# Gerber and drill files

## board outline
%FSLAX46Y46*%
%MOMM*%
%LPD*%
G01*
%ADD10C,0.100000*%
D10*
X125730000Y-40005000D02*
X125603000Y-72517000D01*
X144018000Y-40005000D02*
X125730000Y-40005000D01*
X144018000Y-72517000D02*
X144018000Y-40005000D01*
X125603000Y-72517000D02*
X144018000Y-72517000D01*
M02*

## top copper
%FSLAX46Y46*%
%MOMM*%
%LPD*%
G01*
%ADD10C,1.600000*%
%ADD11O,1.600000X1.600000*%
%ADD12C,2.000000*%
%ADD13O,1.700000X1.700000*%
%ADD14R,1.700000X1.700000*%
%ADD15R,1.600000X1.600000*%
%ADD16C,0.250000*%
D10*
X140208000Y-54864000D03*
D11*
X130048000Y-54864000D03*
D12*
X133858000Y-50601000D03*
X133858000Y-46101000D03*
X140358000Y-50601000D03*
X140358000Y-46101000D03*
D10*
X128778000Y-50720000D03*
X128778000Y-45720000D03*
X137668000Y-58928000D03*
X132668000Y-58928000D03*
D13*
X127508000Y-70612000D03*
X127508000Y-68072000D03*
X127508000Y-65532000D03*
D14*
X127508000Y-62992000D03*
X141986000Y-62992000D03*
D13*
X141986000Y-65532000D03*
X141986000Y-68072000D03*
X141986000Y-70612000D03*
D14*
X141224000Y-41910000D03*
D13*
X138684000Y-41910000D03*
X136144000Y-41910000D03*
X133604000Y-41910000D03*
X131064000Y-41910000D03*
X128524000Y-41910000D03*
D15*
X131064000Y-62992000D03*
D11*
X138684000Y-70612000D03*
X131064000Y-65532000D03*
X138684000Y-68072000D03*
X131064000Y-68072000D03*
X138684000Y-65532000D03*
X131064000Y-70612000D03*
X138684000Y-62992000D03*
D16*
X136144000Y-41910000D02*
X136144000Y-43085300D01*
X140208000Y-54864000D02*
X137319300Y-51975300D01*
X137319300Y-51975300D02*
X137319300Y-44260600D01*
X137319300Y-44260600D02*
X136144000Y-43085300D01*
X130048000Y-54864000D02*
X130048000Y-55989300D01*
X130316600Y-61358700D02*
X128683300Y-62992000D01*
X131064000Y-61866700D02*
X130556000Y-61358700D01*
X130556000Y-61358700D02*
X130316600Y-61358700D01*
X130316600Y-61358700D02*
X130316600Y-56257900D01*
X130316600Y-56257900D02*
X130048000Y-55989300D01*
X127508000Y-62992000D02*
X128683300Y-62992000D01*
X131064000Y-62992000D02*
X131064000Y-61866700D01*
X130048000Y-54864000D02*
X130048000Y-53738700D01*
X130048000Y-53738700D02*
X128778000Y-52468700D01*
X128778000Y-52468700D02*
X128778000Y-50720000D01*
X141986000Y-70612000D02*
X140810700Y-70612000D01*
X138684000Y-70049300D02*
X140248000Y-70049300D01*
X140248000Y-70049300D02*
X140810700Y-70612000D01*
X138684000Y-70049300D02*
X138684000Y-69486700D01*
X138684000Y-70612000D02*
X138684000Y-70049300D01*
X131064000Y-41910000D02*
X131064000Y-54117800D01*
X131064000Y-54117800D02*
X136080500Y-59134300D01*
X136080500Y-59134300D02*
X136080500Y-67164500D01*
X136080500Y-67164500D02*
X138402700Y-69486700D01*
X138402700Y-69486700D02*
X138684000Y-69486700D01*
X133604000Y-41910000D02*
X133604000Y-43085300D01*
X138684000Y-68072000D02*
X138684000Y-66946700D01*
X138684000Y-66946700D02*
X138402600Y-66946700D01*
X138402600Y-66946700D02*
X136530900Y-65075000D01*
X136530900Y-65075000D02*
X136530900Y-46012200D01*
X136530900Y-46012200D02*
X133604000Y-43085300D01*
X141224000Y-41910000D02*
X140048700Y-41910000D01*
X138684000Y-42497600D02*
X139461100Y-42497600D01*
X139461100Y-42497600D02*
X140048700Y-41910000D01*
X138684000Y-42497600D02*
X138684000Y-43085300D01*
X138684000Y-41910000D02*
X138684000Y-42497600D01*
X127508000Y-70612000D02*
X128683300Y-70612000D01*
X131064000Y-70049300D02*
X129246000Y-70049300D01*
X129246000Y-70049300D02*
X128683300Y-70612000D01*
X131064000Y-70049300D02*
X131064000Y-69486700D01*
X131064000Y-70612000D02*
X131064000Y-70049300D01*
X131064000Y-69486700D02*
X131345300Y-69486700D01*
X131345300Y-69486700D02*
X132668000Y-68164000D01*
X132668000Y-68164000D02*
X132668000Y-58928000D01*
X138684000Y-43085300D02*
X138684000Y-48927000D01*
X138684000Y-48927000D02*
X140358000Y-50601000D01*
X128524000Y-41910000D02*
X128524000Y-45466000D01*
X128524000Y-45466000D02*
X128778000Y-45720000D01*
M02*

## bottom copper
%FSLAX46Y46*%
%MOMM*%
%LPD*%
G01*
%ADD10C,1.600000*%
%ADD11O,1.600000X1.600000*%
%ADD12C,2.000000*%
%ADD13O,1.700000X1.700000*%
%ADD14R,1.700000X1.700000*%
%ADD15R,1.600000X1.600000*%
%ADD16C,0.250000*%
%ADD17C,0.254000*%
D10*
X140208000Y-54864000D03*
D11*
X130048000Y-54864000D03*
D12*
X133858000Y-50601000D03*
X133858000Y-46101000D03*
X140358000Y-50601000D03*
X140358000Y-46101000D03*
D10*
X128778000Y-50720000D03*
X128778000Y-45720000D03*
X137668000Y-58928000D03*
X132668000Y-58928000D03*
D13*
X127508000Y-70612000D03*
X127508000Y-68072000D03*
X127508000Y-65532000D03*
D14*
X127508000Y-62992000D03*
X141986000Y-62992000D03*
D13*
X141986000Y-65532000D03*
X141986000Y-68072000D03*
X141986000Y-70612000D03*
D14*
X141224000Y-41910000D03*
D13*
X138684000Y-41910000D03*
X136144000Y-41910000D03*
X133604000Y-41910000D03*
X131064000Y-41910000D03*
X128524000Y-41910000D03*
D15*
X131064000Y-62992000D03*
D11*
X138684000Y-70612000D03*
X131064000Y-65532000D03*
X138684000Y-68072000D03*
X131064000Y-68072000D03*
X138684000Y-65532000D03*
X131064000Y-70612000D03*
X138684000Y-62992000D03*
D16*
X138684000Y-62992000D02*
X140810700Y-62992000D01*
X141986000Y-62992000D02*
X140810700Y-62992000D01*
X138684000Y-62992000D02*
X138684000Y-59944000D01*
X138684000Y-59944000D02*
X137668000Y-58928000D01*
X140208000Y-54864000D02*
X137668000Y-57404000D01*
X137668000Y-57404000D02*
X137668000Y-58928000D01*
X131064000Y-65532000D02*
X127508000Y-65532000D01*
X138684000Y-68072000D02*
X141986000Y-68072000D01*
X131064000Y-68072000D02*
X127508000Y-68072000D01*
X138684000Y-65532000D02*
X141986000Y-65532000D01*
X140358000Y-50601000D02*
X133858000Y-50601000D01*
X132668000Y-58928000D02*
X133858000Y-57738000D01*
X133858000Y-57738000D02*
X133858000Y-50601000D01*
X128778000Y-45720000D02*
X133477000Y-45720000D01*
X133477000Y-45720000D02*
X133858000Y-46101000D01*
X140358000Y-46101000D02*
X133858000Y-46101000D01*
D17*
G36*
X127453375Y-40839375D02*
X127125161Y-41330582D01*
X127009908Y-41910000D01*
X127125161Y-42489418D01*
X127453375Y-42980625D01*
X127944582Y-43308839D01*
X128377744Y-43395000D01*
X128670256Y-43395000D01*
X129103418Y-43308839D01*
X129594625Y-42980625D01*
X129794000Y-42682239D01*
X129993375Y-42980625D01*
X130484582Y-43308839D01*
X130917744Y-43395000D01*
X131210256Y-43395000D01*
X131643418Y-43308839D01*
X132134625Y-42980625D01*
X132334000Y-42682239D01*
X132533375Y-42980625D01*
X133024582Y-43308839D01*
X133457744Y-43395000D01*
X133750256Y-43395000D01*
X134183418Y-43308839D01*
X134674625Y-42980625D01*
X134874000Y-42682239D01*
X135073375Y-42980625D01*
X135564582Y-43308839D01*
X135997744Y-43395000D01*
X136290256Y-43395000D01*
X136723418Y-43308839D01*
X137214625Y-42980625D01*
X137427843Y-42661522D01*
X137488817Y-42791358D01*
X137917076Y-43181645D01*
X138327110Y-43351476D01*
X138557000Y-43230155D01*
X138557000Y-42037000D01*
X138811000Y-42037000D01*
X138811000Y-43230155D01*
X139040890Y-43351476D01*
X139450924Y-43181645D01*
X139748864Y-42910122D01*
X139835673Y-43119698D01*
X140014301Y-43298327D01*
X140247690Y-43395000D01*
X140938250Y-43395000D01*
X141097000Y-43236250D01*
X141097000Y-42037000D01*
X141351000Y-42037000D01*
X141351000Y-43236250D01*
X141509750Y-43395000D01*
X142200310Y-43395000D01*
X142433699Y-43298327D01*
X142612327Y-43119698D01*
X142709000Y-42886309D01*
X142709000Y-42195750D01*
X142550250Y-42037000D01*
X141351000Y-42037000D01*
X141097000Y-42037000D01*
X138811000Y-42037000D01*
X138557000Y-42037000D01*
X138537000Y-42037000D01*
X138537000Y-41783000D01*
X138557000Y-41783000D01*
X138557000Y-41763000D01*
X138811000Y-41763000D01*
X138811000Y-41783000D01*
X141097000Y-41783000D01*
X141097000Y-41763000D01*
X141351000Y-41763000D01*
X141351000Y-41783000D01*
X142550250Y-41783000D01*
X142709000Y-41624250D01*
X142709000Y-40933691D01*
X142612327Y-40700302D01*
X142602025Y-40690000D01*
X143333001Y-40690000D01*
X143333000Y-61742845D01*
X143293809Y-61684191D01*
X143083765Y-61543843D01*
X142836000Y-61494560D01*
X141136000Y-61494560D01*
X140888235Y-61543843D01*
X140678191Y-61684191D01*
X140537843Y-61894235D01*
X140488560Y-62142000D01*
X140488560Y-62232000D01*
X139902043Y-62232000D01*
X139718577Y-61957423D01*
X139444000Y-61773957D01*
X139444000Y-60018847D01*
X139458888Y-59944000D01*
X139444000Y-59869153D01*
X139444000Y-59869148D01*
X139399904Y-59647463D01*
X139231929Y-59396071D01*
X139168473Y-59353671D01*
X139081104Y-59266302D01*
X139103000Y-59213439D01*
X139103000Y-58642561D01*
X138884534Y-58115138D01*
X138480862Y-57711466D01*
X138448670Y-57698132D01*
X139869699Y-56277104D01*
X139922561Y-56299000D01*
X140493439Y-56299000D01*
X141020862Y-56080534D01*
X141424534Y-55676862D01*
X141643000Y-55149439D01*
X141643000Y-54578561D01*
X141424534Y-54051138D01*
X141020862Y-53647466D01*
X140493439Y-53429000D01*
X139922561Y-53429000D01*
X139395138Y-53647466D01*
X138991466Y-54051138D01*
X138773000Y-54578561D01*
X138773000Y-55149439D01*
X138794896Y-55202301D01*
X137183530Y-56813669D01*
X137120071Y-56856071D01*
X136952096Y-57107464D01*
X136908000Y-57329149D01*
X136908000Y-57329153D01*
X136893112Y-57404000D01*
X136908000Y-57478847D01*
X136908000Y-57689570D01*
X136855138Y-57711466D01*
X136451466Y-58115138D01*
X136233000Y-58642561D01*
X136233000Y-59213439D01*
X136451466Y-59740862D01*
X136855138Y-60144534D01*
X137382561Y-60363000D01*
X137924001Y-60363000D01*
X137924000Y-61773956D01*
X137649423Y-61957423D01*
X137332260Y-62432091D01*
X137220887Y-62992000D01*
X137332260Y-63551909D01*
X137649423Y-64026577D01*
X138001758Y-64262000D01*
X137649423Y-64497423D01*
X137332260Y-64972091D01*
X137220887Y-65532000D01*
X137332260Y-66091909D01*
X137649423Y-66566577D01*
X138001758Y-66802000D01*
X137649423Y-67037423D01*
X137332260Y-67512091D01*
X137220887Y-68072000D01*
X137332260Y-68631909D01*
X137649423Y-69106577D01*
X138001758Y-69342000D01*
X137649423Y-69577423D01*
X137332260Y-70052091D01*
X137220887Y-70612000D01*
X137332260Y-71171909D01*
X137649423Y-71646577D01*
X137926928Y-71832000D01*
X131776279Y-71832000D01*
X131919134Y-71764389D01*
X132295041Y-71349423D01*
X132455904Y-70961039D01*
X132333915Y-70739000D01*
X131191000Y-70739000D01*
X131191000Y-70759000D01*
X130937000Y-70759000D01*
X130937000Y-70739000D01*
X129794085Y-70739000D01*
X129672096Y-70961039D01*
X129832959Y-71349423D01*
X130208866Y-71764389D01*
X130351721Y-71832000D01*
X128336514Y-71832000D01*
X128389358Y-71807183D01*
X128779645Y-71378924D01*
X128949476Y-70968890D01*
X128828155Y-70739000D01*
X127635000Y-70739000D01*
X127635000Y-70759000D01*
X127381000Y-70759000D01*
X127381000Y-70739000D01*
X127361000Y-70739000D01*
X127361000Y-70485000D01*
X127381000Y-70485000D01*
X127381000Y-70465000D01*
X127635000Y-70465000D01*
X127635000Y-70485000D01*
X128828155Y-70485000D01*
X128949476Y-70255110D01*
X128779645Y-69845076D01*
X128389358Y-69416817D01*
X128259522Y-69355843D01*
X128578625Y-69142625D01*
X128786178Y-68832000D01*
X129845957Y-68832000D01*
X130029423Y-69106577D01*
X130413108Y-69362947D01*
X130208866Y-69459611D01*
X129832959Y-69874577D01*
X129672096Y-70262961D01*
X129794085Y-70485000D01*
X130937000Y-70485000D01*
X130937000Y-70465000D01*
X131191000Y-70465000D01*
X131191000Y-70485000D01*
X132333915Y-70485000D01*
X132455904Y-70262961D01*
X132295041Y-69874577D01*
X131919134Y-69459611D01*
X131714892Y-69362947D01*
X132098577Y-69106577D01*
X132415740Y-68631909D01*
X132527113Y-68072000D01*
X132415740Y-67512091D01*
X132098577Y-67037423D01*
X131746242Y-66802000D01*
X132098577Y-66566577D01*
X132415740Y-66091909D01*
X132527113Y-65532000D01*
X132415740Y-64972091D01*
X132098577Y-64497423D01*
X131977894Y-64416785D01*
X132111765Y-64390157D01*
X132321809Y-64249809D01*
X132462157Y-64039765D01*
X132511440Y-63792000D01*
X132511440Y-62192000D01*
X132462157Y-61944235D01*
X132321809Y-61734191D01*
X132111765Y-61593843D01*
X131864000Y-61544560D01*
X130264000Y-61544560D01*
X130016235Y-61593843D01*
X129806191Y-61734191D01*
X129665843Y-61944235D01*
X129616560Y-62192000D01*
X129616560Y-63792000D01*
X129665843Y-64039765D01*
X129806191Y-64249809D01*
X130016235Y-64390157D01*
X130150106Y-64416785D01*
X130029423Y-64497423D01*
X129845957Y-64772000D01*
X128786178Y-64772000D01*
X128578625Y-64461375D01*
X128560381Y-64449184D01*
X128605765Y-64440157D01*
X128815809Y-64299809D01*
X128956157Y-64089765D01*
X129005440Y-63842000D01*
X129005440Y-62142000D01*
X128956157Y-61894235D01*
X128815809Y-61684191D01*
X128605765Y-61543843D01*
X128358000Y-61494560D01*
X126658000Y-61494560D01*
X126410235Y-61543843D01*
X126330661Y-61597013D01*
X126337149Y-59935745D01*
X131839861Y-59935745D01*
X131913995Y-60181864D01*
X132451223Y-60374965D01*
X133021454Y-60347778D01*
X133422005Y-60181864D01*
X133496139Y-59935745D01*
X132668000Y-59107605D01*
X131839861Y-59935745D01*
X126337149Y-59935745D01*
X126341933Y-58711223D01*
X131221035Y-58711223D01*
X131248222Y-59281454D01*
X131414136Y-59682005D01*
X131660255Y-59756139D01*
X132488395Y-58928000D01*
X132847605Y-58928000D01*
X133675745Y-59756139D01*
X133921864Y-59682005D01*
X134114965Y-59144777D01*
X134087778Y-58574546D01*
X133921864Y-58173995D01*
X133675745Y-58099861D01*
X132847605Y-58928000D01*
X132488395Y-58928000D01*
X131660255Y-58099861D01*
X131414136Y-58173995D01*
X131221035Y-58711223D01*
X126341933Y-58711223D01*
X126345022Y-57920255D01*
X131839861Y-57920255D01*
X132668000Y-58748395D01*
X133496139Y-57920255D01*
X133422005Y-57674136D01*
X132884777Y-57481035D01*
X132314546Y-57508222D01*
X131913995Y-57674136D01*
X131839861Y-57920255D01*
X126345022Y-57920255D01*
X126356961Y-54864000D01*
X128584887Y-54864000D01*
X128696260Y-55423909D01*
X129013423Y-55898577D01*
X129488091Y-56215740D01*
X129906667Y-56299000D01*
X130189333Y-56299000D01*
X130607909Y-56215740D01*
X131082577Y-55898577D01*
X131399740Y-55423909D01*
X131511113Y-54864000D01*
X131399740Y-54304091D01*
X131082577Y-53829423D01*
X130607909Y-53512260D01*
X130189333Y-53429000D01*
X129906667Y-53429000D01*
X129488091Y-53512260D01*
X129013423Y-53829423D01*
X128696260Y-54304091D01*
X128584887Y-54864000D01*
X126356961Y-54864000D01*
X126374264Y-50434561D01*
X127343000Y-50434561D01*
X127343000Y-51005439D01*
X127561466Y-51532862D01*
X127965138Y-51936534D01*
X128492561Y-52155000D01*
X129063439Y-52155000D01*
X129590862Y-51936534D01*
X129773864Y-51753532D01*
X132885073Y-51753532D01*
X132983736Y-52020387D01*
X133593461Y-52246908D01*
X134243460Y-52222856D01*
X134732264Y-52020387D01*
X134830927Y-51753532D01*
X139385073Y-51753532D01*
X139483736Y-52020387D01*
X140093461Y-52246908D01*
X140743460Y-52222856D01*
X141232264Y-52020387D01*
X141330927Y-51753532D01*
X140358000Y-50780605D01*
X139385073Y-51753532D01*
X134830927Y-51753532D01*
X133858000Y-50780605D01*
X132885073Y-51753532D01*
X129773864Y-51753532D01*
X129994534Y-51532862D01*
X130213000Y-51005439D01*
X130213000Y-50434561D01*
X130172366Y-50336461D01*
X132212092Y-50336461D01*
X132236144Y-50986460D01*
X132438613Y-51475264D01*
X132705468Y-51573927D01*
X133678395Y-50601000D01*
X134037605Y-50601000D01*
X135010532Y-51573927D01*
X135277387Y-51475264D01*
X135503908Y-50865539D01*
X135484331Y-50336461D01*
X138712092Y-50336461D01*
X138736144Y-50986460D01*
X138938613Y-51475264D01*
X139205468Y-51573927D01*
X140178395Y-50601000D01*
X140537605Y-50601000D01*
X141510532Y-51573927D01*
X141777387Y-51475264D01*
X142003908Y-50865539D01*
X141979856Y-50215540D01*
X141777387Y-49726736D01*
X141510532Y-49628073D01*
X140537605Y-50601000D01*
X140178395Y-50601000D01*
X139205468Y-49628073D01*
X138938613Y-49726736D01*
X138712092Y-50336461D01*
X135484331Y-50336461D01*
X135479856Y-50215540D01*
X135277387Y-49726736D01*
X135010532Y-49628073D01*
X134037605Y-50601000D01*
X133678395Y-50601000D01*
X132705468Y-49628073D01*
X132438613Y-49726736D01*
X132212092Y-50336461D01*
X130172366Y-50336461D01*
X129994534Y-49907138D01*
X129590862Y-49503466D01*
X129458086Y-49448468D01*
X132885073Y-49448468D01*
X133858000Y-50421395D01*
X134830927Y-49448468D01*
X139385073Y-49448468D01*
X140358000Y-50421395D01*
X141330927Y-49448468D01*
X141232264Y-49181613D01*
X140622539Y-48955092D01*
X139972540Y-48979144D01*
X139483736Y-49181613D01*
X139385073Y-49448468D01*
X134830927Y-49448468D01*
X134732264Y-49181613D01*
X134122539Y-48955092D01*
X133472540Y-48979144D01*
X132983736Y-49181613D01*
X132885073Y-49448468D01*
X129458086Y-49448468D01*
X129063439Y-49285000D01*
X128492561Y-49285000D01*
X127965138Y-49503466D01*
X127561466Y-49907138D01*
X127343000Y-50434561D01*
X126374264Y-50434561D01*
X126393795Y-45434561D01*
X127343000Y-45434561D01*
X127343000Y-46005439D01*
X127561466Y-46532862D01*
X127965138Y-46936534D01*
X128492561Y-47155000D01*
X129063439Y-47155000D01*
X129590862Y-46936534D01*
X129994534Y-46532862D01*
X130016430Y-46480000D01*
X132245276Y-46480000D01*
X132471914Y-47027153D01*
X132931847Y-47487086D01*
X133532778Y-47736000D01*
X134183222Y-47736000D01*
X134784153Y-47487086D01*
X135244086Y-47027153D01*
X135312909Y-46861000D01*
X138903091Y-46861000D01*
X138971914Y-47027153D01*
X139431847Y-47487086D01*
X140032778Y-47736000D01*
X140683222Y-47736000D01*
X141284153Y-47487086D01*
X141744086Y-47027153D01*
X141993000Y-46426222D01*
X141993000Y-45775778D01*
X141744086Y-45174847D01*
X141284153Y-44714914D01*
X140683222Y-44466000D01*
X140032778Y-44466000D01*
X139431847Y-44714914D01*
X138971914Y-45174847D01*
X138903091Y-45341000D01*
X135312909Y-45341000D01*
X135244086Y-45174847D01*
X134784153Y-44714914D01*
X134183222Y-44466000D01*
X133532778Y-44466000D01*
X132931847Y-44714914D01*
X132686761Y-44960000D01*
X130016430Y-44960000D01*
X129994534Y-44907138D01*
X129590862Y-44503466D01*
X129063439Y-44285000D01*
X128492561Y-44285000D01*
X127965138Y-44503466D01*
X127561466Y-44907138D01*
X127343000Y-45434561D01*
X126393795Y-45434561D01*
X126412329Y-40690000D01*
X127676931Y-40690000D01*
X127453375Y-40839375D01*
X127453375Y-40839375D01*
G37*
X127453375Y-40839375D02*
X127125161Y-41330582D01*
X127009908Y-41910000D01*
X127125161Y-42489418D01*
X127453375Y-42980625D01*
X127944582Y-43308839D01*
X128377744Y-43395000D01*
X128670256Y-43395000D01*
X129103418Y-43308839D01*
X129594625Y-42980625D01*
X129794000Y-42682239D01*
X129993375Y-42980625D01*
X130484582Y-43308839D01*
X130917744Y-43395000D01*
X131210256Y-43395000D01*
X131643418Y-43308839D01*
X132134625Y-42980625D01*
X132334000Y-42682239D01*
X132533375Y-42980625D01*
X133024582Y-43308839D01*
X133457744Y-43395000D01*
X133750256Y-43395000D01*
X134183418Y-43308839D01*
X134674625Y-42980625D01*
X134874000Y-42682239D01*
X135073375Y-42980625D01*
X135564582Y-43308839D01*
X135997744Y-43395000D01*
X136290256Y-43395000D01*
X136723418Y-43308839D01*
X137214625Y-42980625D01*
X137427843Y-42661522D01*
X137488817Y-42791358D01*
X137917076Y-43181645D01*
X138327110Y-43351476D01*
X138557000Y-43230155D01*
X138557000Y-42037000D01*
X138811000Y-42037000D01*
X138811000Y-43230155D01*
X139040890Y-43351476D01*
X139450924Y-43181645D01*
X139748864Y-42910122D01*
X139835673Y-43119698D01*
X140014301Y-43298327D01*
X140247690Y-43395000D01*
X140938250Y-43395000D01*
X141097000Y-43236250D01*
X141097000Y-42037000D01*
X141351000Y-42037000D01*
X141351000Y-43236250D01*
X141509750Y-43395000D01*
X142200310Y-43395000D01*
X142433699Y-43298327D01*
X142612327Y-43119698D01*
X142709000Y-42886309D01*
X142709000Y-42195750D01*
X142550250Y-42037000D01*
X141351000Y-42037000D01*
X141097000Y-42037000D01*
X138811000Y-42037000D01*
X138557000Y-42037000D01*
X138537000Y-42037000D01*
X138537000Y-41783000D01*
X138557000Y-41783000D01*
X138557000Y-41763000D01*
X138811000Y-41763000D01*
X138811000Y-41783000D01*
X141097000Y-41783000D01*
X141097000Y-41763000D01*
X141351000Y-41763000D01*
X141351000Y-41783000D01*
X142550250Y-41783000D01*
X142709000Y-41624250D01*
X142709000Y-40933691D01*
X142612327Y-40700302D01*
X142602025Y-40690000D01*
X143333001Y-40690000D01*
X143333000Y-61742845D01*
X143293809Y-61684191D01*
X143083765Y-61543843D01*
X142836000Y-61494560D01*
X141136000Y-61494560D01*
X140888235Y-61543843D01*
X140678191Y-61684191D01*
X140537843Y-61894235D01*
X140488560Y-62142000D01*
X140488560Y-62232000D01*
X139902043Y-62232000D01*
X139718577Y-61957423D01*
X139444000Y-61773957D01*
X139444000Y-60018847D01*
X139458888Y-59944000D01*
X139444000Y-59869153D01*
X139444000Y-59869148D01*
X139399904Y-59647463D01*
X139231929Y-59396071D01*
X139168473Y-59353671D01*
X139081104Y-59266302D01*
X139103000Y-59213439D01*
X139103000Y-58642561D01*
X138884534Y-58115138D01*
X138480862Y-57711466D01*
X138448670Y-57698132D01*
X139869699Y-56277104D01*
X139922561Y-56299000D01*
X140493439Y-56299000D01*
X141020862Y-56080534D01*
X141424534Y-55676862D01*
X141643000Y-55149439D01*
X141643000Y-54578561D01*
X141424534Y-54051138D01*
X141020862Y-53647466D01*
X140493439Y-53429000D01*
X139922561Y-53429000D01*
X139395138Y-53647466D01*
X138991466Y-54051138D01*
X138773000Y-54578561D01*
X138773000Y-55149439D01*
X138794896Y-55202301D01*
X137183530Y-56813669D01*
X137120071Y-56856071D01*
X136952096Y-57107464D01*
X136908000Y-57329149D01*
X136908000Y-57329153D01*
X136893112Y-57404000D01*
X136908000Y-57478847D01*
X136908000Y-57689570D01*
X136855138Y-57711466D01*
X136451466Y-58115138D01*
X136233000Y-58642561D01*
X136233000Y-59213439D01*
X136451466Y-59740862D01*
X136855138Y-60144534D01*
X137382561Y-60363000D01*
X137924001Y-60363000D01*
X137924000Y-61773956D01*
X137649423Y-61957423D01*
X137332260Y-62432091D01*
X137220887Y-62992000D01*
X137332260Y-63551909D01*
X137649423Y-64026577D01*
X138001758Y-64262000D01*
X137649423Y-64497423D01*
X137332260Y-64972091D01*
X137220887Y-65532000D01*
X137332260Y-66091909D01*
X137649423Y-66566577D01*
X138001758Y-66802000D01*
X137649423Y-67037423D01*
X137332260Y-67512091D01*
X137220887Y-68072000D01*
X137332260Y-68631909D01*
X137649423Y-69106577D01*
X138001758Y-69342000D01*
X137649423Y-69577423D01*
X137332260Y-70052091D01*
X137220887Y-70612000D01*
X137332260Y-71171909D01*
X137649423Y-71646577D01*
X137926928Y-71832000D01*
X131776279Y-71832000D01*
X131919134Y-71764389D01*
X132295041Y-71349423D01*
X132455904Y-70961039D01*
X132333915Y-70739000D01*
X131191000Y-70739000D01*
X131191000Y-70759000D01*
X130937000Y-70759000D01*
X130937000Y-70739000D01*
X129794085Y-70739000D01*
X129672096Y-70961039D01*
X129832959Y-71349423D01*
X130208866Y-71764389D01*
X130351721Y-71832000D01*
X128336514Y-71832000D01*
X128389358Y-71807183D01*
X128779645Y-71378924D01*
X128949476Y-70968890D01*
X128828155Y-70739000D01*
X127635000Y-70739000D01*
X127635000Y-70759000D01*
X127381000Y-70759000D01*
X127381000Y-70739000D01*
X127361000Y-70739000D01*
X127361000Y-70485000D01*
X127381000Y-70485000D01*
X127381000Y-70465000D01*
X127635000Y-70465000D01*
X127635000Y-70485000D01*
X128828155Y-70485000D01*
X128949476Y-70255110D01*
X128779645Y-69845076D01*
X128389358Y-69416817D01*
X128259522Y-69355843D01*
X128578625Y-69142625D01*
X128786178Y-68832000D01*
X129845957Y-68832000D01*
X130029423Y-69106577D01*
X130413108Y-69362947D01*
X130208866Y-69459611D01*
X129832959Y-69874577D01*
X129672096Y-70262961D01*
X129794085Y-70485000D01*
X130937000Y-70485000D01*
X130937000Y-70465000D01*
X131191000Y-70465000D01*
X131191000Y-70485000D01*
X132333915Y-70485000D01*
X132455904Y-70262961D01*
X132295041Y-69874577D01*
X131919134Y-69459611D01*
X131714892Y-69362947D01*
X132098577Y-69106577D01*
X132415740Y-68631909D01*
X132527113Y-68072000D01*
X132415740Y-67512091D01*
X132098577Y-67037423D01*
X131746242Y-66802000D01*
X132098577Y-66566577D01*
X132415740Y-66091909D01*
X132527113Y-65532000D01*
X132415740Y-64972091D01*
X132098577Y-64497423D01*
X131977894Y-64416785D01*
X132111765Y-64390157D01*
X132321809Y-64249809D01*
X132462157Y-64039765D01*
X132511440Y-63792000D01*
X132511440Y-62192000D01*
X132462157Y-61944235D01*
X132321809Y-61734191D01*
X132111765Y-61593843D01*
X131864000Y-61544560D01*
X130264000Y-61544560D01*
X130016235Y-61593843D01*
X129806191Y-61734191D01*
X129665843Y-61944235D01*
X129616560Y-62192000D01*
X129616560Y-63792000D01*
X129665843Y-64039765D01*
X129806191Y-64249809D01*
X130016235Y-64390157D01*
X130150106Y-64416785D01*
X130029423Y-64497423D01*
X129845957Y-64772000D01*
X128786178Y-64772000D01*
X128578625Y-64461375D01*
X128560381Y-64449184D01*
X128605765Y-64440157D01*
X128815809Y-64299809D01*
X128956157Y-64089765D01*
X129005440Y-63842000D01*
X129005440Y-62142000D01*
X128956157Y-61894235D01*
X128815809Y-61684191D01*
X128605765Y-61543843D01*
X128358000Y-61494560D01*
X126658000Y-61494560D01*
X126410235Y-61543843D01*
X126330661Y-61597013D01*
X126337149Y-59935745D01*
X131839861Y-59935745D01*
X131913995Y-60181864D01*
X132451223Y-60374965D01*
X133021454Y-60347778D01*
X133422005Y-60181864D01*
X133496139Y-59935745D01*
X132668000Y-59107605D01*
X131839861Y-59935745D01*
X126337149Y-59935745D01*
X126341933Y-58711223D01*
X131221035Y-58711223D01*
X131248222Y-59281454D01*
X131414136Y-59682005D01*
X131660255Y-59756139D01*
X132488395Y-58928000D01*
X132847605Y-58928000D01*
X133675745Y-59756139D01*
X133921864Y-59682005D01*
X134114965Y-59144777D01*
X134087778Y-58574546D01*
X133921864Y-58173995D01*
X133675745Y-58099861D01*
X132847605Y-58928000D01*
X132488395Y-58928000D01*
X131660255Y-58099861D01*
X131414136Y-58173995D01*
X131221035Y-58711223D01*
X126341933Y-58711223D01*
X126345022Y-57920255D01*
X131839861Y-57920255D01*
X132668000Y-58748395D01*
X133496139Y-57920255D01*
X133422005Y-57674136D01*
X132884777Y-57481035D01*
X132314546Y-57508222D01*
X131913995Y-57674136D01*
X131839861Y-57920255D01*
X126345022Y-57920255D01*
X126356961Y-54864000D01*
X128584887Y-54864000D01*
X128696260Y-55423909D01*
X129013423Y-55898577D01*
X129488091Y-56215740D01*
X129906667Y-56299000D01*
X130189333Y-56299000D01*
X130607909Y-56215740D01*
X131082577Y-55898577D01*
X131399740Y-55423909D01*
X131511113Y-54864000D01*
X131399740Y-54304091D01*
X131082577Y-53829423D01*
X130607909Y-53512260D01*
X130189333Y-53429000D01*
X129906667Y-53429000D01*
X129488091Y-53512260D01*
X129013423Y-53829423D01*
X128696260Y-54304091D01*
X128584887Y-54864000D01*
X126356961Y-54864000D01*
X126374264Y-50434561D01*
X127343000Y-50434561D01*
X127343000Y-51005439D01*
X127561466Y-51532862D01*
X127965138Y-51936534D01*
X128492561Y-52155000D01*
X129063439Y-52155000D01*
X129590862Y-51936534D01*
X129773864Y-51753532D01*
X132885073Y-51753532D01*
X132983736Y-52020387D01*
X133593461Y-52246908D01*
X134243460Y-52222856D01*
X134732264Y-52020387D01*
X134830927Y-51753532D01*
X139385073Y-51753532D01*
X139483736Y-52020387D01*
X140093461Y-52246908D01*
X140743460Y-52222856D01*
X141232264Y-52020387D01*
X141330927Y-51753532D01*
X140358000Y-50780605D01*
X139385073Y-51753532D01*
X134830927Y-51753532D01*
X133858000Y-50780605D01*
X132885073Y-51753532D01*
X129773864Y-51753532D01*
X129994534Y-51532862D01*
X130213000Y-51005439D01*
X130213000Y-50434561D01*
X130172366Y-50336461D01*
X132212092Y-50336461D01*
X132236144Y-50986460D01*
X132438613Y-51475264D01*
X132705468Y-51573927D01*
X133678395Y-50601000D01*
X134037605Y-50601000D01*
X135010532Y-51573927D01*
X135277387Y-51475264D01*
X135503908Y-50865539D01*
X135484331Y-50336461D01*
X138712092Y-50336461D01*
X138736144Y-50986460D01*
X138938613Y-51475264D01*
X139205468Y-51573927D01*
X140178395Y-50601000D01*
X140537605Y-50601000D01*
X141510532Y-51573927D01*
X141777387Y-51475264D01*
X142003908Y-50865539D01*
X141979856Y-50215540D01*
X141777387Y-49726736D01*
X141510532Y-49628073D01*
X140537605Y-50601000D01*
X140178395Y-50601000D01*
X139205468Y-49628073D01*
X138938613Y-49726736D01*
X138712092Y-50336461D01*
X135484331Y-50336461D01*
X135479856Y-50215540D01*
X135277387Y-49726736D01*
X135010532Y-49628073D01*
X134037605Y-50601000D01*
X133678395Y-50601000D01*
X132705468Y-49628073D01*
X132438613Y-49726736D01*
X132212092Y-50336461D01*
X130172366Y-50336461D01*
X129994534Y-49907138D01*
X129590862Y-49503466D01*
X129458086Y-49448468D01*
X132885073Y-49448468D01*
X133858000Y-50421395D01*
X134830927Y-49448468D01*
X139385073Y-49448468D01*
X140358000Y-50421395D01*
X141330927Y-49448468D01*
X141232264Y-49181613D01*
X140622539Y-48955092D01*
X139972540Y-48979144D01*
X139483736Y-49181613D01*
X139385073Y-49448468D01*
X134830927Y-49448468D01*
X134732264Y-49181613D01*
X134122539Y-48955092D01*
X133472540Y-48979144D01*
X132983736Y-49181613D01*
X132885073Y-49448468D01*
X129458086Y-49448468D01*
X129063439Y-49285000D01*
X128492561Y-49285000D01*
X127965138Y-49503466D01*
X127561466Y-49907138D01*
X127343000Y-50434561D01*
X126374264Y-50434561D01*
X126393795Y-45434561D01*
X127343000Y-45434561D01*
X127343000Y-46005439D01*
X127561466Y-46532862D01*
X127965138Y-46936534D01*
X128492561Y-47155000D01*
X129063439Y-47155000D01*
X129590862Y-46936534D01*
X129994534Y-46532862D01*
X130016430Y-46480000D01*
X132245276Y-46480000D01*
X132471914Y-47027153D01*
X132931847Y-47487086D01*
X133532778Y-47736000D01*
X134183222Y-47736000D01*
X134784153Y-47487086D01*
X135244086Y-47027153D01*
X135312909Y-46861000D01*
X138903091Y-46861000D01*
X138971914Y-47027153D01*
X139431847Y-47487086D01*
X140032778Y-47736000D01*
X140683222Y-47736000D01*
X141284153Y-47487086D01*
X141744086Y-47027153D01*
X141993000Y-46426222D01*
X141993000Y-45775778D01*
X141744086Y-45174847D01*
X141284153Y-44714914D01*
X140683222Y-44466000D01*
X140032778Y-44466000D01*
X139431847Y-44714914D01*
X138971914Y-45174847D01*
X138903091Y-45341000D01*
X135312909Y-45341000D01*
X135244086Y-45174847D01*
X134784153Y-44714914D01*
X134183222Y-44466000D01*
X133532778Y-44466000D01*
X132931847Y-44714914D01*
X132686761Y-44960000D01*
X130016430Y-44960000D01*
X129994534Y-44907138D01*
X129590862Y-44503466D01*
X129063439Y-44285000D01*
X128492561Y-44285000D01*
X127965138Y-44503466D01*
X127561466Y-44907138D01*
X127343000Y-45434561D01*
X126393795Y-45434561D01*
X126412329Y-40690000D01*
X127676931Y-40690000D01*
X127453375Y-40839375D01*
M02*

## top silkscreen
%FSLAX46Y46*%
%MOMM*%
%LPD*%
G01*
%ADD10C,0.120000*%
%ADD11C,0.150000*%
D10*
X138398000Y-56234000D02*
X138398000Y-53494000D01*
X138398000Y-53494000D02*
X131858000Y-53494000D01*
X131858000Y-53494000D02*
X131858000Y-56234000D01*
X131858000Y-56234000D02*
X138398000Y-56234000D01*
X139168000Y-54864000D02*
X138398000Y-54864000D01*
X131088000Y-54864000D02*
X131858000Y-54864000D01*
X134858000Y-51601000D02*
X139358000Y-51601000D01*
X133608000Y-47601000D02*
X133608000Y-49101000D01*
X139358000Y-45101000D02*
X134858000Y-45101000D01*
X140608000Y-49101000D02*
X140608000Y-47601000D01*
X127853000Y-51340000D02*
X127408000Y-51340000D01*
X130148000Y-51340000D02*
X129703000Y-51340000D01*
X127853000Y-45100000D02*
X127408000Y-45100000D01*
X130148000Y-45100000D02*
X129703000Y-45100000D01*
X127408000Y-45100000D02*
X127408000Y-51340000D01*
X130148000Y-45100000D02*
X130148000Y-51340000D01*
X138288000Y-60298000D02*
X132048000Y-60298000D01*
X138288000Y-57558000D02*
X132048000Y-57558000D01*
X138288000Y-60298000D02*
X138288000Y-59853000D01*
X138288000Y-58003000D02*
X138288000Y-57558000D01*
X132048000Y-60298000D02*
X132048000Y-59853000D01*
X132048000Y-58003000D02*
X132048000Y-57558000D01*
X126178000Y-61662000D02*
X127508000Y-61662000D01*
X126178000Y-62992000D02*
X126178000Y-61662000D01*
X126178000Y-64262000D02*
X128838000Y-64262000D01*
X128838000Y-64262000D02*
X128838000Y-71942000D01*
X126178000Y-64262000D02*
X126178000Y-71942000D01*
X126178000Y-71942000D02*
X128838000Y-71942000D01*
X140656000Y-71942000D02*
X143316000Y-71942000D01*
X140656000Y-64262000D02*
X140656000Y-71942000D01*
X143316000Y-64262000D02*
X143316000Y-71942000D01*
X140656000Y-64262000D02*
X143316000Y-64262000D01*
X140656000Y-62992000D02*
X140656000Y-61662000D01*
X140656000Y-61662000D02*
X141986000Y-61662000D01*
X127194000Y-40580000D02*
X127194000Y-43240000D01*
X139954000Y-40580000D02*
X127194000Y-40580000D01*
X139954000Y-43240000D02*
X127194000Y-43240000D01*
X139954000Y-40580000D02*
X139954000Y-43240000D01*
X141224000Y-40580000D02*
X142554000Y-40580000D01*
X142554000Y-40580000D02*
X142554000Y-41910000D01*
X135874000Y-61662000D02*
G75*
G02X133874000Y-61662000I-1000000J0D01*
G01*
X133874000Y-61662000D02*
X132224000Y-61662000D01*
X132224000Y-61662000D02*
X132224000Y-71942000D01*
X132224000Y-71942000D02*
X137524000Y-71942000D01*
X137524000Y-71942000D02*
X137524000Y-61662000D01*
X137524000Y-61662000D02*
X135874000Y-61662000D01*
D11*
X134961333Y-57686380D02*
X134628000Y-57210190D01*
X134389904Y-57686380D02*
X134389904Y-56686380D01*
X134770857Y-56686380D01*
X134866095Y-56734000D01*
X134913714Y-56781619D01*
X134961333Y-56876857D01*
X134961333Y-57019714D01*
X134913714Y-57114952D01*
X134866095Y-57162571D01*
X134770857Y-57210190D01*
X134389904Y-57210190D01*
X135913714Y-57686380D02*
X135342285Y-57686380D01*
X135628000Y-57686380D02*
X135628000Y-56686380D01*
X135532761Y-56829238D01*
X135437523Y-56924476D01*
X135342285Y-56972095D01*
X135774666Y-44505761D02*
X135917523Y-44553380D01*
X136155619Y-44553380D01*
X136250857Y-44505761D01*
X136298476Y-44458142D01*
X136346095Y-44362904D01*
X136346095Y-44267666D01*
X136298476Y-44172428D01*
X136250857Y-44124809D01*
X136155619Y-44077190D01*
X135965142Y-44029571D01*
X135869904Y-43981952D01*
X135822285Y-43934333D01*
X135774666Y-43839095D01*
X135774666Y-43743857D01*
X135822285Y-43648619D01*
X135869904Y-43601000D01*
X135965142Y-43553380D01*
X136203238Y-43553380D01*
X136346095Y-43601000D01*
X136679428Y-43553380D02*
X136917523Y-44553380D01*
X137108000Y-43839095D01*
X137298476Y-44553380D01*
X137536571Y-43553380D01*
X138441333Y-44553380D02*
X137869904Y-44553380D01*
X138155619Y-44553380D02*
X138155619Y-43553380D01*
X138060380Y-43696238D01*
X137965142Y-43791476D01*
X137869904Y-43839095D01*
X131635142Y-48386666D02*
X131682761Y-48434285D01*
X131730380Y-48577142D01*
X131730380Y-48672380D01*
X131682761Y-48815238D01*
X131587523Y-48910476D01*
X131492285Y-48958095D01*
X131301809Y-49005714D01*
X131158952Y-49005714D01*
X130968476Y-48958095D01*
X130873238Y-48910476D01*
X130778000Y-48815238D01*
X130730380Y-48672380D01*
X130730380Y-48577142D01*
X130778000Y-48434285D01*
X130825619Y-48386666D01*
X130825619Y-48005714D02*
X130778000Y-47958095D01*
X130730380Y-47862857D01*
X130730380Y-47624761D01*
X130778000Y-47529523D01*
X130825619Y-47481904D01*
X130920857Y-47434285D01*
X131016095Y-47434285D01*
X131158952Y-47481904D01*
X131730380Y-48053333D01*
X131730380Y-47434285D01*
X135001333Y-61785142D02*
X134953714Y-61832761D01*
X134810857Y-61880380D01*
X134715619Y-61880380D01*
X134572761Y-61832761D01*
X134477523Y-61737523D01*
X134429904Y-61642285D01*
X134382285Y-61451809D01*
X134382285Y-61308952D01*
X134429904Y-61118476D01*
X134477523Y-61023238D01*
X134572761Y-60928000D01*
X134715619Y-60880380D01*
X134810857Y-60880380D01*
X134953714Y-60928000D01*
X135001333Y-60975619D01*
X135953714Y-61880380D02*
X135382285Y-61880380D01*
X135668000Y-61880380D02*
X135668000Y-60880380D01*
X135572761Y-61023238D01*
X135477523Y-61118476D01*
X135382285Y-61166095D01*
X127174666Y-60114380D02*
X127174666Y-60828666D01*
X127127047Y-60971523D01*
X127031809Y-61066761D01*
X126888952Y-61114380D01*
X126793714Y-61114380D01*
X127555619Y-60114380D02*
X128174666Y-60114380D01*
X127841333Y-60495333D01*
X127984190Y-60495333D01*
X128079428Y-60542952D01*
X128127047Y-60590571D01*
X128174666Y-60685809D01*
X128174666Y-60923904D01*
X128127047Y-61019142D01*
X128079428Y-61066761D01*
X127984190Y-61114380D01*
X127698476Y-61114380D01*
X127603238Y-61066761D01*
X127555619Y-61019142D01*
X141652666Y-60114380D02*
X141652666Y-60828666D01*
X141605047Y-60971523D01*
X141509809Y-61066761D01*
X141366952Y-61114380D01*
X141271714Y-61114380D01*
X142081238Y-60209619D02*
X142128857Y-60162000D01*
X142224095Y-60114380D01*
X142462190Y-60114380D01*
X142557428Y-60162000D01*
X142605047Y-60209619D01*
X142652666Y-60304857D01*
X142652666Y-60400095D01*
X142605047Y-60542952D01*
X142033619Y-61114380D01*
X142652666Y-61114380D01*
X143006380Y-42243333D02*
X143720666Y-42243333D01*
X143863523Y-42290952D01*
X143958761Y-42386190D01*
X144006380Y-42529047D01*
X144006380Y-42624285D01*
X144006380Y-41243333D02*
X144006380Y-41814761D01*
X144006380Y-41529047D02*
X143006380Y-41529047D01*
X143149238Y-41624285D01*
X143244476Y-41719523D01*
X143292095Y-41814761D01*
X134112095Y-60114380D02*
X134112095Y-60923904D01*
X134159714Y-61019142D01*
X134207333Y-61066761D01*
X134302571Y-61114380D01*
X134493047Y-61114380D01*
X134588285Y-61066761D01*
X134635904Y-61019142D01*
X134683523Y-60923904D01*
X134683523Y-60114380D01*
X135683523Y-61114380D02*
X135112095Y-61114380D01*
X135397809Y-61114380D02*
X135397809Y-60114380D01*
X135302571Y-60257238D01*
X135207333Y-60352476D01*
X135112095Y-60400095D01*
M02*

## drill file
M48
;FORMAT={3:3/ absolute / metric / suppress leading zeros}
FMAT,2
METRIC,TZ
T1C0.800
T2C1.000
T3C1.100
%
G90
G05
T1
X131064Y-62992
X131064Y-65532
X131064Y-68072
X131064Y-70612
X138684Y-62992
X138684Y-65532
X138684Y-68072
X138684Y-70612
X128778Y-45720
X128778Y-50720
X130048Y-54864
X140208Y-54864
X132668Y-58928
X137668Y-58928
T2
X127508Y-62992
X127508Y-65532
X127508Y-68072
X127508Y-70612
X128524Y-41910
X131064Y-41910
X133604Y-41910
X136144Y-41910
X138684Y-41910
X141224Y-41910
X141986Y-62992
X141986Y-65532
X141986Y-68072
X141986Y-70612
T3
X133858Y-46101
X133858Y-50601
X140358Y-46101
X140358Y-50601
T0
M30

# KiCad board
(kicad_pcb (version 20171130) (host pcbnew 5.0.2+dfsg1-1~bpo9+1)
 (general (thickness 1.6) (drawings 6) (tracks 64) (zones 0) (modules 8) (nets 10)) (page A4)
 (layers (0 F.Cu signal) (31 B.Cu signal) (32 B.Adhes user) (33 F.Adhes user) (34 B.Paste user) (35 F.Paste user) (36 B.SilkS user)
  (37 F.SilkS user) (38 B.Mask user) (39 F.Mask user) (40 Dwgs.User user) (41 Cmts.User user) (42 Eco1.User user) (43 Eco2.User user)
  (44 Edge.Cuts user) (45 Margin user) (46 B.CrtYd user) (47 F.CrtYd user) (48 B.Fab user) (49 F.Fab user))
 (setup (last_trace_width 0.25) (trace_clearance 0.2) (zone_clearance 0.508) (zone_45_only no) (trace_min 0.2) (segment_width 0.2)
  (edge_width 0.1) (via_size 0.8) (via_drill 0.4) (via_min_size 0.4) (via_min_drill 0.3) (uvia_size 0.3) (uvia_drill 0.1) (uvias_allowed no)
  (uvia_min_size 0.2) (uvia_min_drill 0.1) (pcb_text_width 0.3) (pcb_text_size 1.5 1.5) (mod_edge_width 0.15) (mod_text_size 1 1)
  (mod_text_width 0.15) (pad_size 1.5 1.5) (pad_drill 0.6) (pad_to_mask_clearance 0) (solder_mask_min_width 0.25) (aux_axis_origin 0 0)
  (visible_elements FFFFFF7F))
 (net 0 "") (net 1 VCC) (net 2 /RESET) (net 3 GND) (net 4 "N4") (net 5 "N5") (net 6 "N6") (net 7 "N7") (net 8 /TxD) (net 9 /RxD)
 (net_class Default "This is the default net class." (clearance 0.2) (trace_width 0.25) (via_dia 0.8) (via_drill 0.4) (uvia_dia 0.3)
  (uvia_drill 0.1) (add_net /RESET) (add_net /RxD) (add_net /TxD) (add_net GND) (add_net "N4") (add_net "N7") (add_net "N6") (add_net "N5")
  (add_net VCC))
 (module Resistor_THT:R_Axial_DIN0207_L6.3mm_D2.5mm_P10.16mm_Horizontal (layer F.Cu) (at 140.208 54.864 180)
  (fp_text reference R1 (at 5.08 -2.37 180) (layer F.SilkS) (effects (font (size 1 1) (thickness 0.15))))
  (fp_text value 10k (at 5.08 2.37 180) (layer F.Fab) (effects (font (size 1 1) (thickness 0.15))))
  (fp_line (start 1.81 -1.37) (end 1.81 1.37) (layer F.SilkS) (width 0.12))
  (fp_line (start 1.81 1.37) (end 8.35 1.37) (layer F.SilkS) (width 0.12))
  (fp_line (start 8.35 1.37) (end 8.35 -1.37) (layer F.SilkS) (width 0.12))
  (fp_line (start 8.35 -1.37) (end 1.81 -1.37) (layer F.SilkS) (width 0.12))
  (fp_line (start 1.04 0) (end 1.81 0) (layer F.SilkS) (width 0.12))
  (fp_line (start 9.12 0) (end 8.35 0) (layer F.SilkS) (width 0.12))
  (pad 1 thru_hole circle (at 0 0 180) (size 1.6 1.6) (drill 0.8) (layers *.Cu *.Mask) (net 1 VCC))
  (pad 2 thru_hole oval (at 10.16 0 180) (size 1.6 1.6) (drill 0.8) (layers *.Cu *.Mask) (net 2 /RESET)))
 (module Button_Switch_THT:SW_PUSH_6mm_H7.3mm (layer F.Cu) (at 133.858 46.101)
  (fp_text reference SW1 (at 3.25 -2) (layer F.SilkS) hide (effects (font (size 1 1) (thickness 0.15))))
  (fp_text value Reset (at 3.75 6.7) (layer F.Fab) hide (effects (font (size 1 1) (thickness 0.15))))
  (fp_line (start 1 5.5) (end 5.5 5.5) (layer F.SilkS) (width 0.12))
  (fp_line (start -0.25 1.5) (end -0.25 3) (layer F.SilkS) (width 0.12))
  (fp_line (start 5.5 -1) (end 1 -1) (layer F.SilkS) (width 0.12))
  (fp_line (start 6.75 3) (end 6.75 1.5) (layer F.SilkS) (width 0.12))
  (pad 2 thru_hole circle (at 0 4.5 90) (size 2 2) (drill 1.1) (layers *.Cu *.Mask) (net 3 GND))
  (pad 1 thru_hole circle (at 0 0 90) (size 2 2) (drill 1.1) (layers *.Cu *.Mask) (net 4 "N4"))
  (pad 2 thru_hole circle (at 6.5 4.5 90) (size 2 2) (drill 1.1) (layers *.Cu *.Mask) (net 3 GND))
  (pad 1 thru_hole circle (at 6.5 0 90) (size 2 2) (drill 1.1) (layers *.Cu *.Mask) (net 4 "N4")))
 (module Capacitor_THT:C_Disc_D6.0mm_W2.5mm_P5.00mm (layer F.Cu) (at 128.778 45.72 270)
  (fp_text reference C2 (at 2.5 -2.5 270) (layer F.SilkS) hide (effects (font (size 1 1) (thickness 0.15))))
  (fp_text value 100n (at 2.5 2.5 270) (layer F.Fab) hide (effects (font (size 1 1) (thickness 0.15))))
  (fp_line (start 5.62 0.925) (end 5.62 1.37) (layer F.SilkS) (width 0.12))
  (fp_line (start 5.62 -1.37) (end 5.62 -0.925) (layer F.SilkS) (width 0.12))
  (fp_line (start -0.62 0.925) (end -0.62 1.37) (layer F.SilkS) (width 0.12))
  (fp_line (start -0.62 -1.37) (end -0.62 -0.925) (layer F.SilkS) (width 0.12))
  (fp_line (start -0.62 1.37) (end 5.62 1.37) (layer F.SilkS) (width 0.12))
  (fp_line (start -0.62 -1.37) (end 5.62 -1.37) (layer F.SilkS) (width 0.12))
  (pad 2 thru_hole circle (at 5 0 270) (size 1.6 1.6) (drill 0.8) (layers *.Cu *.Mask) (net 2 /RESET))
  (pad 1 thru_hole circle (at 0 0 270) (size 1.6 1.6) (drill 0.8) (layers *.Cu *.Mask) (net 4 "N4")))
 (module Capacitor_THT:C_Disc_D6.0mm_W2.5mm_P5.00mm (layer F.Cu) (at 137.668 58.928 180)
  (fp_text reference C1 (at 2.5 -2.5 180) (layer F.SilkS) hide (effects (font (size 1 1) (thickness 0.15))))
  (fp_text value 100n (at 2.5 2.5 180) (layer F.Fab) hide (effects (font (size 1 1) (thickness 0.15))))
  (fp_line (start -0.62 -1.37) (end 5.62 -1.37) (layer F.SilkS) (width 0.12))
  (fp_line (start -0.62 1.37) (end 5.62 1.37) (layer F.SilkS) (width 0.12))
  (fp_line (start -0.62 -1.37) (end -0.62 -0.925) (layer F.SilkS) (width 0.12))
  (fp_line (start -0.62 0.925) (end -0.62 1.37) (layer F.SilkS) (width 0.12))
  (fp_line (start 5.62 -1.37) (end 5.62 -0.925) (layer F.SilkS) (width 0.12))
  (fp_line (start 5.62 0.925) (end 5.62 1.37) (layer F.SilkS) (width 0.12))
  (pad 1 thru_hole circle (at 0 0 180) (size 1.6 1.6) (drill 0.8) (layers *.Cu *.Mask) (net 1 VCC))
  (pad 2 thru_hole circle (at 5 0 180) (size 1.6 1.6) (drill 0.8) (layers *.Cu *.Mask) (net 3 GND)))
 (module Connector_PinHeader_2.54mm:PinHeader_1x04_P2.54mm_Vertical (layer F.Cu) (at 127.508 62.992)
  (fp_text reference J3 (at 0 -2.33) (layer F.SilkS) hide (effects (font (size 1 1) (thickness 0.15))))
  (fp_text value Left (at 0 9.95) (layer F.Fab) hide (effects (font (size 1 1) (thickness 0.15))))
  (fp_line (start -1.33 -1.33) (end 0 -1.33) (layer F.SilkS) (width 0.12))
  (fp_line (start -1.33 0) (end -1.33 -1.33) (layer F.SilkS) (width 0.12))
  (fp_line (start -1.33 1.27) (end 1.33 1.27) (layer F.SilkS) (width 0.12))
  (fp_line (start 1.33 1.27) (end 1.33 8.95) (layer F.SilkS) (width 0.12))
  (fp_line (start -1.33 1.27) (end -1.33 8.95) (layer F.SilkS) (width 0.12))
  (fp_line (start -1.33 8.95) (end 1.33 8.95) (layer F.SilkS) (width 0.12))
  (pad 4 thru_hole oval (at 0 7.62) (size 1.7 1.7) (drill 1) (layers *.Cu *.Mask) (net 3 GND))
  (pad 3 thru_hole oval (at 0 5.08) (size 1.7 1.7) (drill 1) (layers *.Cu *.Mask) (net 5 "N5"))
  (pad 2 thru_hole oval (at 0 2.54) (size 1.7 1.7) (drill 1) (layers *.Cu *.Mask) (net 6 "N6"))
  (pad 1 thru_hole rect (at 0 0) (size 1.7 1.7) (drill 1) (layers *.Cu *.Mask) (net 2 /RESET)))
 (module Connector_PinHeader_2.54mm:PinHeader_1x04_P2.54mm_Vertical (layer F.Cu) (at 141.986 62.992)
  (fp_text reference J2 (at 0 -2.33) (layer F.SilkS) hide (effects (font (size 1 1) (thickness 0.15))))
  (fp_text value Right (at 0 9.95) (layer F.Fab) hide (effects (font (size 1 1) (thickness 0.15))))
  (fp_line (start -1.33 8.95) (end 1.33 8.95) (layer F.SilkS) (width 0.12))
  (fp_line (start -1.33 1.27) (end -1.33 8.95) (layer F.SilkS) (width 0.12))
  (fp_line (start 1.33 1.27) (end 1.33 8.95) (layer F.SilkS) (width 0.12))
  (fp_line (start -1.33 1.27) (end 1.33 1.27) (layer F.SilkS) (width 0.12))
  (fp_line (start -1.33 0) (end -1.33 -1.33) (layer F.SilkS) (width 0.12))
  (fp_line (start -1.33 -1.33) (end 0 -1.33) (layer F.SilkS) (width 0.12))
  (pad 1 thru_hole rect (at 0 0) (size 1.7 1.7) (drill 1) (layers *.Cu *.Mask) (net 1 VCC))
  (pad 2 thru_hole oval (at 0 2.54) (size 1.7 1.7) (drill 1) (layers *.Cu *.Mask) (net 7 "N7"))
  (pad 3 thru_hole oval (at 0 5.08) (size 1.7 1.7) (drill 1) (layers *.Cu *.Mask) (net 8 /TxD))
  (pad 4 thru_hole oval (at 0 7.62) (size 1.7 1.7) (drill 1) (layers *.Cu *.Mask) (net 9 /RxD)))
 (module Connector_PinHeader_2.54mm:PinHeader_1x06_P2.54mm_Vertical (layer F.Cu) (at 141.224 41.91 270)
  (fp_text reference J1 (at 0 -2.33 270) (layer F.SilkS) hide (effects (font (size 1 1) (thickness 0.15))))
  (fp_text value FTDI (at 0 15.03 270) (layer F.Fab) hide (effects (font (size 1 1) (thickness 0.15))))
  (fp_line (start -1.33 14.03) (end 1.33 14.03) (layer F.SilkS) (width 0.12))
  (fp_line (start -1.33 1.27) (end -1.33 14.03) (layer F.SilkS) (width 0.12))
  (fp_line (start 1.33 1.27) (end 1.33 14.03) (layer F.SilkS) (width 0.12))
  (fp_line (start -1.33 1.27) (end 1.33 1.27) (layer F.SilkS) (width 0.12))
  (fp_line (start -1.33 0) (end -1.33 -1.33) (layer F.SilkS) (width 0.12))
  (fp_line (start -1.33 -1.33) (end 0 -1.33) (layer F.SilkS) (width 0.12))
  (pad 1 thru_hole rect (at 0 0 270) (size 1.7 1.7) (drill 1) (layers *.Cu *.Mask) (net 3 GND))
  (pad 2 thru_hole oval (at 0 2.54 270) (size 1.7 1.7) (drill 1) (layers *.Cu *.Mask) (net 3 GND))
  (pad 3 thru_hole oval (at 0 5.08 270) (size 1.7 1.7) (drill 1) (layers *.Cu *.Mask) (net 1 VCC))
  (pad 4 thru_hole oval (at 0 7.62 270) (size 1.7 1.7) (drill 1) (layers *.Cu *.Mask) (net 8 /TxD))
  (pad 5 thru_hole oval (at 0 10.16 270) (size 1.7 1.7) (drill 1) (layers *.Cu *.Mask) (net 9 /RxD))
  (pad 6 thru_hole oval (at 0 12.7 270) (size 1.7 1.7) (drill 1) (layers *.Cu *.Mask) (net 4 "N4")))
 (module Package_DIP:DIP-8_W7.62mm (layer F.Cu) (at 131.064 62.992)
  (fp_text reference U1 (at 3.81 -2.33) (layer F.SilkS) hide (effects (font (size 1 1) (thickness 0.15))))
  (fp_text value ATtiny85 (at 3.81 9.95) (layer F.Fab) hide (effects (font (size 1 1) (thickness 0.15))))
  (fp_arc (start 3.81 -1.33) (end 2.81 -1.33) (angle -180) (layer F.SilkS) (width 0.12))
  (fp_line (start 2.81 -1.33) (end 1.16 -1.33) (layer F.SilkS) (width 0.12))
  (fp_line (start 1.16 -1.33) (end 1.16 8.95) (layer F.SilkS) (width 0.12))
  (fp_line (start 1.16 8.95) (end 6.46 8.95) (layer F.SilkS) (width 0.12))
  (fp_line (start 6.46 8.95) (end 6.46 -1.33) (layer F.SilkS) (width 0.12))
  (fp_line (start 6.46 -1.33) (end 4.81 -1.33) (layer F.SilkS) (width 0.12))
  (pad 1 thru_hole rect (at 0 0) (size 1.6 1.6) (drill 0.8) (layers *.Cu *.Mask) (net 2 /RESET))
  (pad 5 thru_hole oval (at 7.62 7.62) (size 1.6 1.6) (drill 0.8) (layers *.Cu *.Mask) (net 9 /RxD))
  (pad 2 thru_hole oval (at 0 2.54) (size 1.6 1.6) (drill 0.8) (layers *.Cu *.Mask) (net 6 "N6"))
  (pad 6 thru_hole oval (at 7.62 5.08) (size 1.6 1.6) (drill 0.8) (layers *.Cu *.Mask) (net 8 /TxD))
  (pad 3 thru_hole oval (at 0 5.08) (size 1.6 1.6) (drill 0.8) (layers *.Cu *.Mask) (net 5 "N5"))
  (pad 7 thru_hole oval (at 7.62 2.54) (size 1.6 1.6) (drill 0.8) (layers *.Cu *.Mask) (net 7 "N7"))
  (pad 4 thru_hole oval (at 0 7.62) (size 1.6 1.6) (drill 0.8) (layers *.Cu *.Mask) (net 3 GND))
  (pad 8 thru_hole oval (at 7.62 0) (size 1.6 1.6) (drill 0.8) (layers *.Cu *.Mask) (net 1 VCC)))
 (gr_line (start 125.73 40.005) (end 125.603 72.517) (layer Edge.Cuts) (width 0.1))
 (gr_line (start 144.018 40.005) (end 125.73 40.005) (layer Edge.Cuts) (width 0.1))
 (gr_line (start 144.018 72.517) (end 144.018 40.005) (layer Edge.Cuts) (width 0.1))
 (gr_line (start 125.603 72.517) (end 144.018 72.517) (layer Edge.Cuts) (width 0.1))
 (segment (start 138.684 62.992) (end 140.8107 62.992) (width 0.25) (layer B.Cu) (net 1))
 (segment (start 141.986 62.992) (end 140.8107 62.992) (width 0.25) (layer B.Cu) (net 1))
 (segment (start 138.684 62.992) (end 138.684 59.944) (width 0.25) (layer B.Cu) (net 1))
 (segment (start 138.684 59.944) (end 137.668 58.928) (width 0.25) (layer B.Cu) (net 1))
 (segment (start 136.144 41.91) (end 136.144 43.0853) (width 0.25) (layer F.Cu) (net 1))
 (segment (start 140.208 54.864) (end 137.3193 51.9753) (width 0.25) (layer F.Cu) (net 1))
 (segment (start 137.3193 51.9753) (end 137.3193 44.2606) (width 0.25) (layer F.Cu) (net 1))
 (segment (start 137.3193 44.2606) (end 136.144 43.0853) (width 0.25) (layer F.Cu) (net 1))
 (segment (start 140.208 54.864) (end 137.668 57.404) (width 0.25) (layer B.Cu) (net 1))
 (segment (start 137.668 57.404) (end 137.668 58.928) (width 0.25) (layer B.Cu) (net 1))
 (segment (start 130.048 54.864) (end 130.048 55.9893) (width 0.25) (layer F.Cu) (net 2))
 (segment (start 130.3166 61.3587) (end 128.6833 62.992) (width 0.25) (layer F.Cu) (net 2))
 (segment (start 131.064 61.8667) (end 130.556 61.3587) (width 0.25) (layer F.Cu) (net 2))
 (segment (start 130.556 61.3587) (end 130.3166 61.3587) (width 0.25) (layer F.Cu) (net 2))
 (segment (start 130.3166 61.3587) (end 130.3166 56.2579) (width 0.25) (layer F.Cu) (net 2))
 (segment (start 130.3166 56.2579) (end 130.048 55.9893) (width 0.25) (layer F.Cu) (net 2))
 (segment (start 127.508 62.992) (end 128.6833 62.992) (width 0.25) (layer F.Cu) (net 2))
 (segment (start 131.064 62.992) (end 131.064 61.8667) (width 0.25) (layer F.Cu) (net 2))
 (segment (start 130.048 54.864) (end 130.048 53.7387) (width 0.25) (layer F.Cu) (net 2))
 (segment (start 130.048 53.7387) (end 128.778 52.4687) (width 0.25) (layer F.Cu) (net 2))
 (segment (start 128.778 52.4687) (end 128.778 50.72) (width 0.25) (layer F.Cu) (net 2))
 (segment (start 141.986 70.612) (end 140.8107 70.612) (width 0.25) (layer F.Cu) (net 9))
 (segment (start 138.684 70.0493) (end 140.248 70.0493) (width 0.25) (layer F.Cu) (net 9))
 (segment (start 140.248 70.0493) (end 140.8107 70.612) (width 0.25) (layer F.Cu) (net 9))
 (segment (start 138.684 70.0493) (end 138.684 69.4867) (width 0.25) (layer F.Cu) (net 9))
 (segment (start 138.684 70.612) (end 138.684 70.0493) (width 0.25) (layer F.Cu) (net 9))
 (segment (start 131.064 41.91) (end 131.064 54.1178) (width 0.25) (layer F.Cu) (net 9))
 (segment (start 131.064 54.1178) (end 136.0805 59.1343) (width 0.25) (layer F.Cu) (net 9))
 (segment (start 136.0805 59.1343) (end 136.0805 67.1645) (width 0.25) (layer F.Cu) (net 9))
 (segment (start 136.0805 67.1645) (end 138.4027 69.4867) (width 0.25) (layer F.Cu) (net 9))
 (segment (start 138.4027 69.4867) (end 138.684 69.4867) (width 0.25) (layer F.Cu) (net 9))
 (segment (start 131.064 65.532) (end 127.508 65.532) (width 0.25) (layer B.Cu) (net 6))
 (segment (start 133.604 41.91) (end 133.604 43.0853) (width 0.25) (layer F.Cu) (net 8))
 (segment (start 138.684 68.072) (end 138.684 66.9467) (width 0.25) (layer F.Cu) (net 8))
 (segment (start 138.684 66.9467) (end 138.4026 66.9467) (width 0.25) (layer F.Cu) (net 8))
 (segment (start 138.4026 66.9467) (end 136.5309 65.075) (width 0.25) (layer F.Cu) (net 8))
 (segment (start 136.5309 65.075) (end 136.5309 46.0122) (width 0.25) (layer F.Cu) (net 8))
 (segment (start 136.5309 46.0122) (end 133.604 43.0853) (width 0.25) (layer F.Cu) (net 8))
 (segment (start 138.684 68.072) (end 141.986 68.072) (width 0.25) (layer B.Cu) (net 8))
 (segment (start 131.064 68.072) (end 127.508 68.072) (width 0.25) (layer B.Cu) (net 5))
 (segment (start 138.684 65.532) (end 141.986 65.532) (width 0.25) (layer B.Cu) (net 7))
 (segment (start 141.224 41.91) (end 140.0487 41.91) (width 0.25) (layer F.Cu) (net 3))
 (segment (start 138.684 42.4976) (end 139.4611 42.4976) (width 0.25) (layer F.Cu) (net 3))
 (segment (start 139.4611 42.4976) (end 140.0487 41.91) (width 0.25) (layer F.Cu) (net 3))
 (segment (start 138.684 42.4976) (end 138.684 43.0853) (width 0.25) (layer F.Cu) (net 3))
 (segment (start 138.684 41.91) (end 138.684 42.4976) (width 0.25) (layer F.Cu) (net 3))
 (segment (start 127.508 70.612) (end 128.6833 70.612) (width 0.25) (layer F.Cu) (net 3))
 (segment (start 131.064 70.0493) (end 129.246 70.0493) (width 0.25) (layer F.Cu) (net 3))
 (segment (start 129.246 70.0493) (end 128.6833 70.612) (width 0.25) (layer F.Cu) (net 3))
 (segment (start 131.064 70.0493) (end 131.064 69.4867) (width 0.25) (layer F.Cu) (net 3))
 (segment (start 131.064 70.612) (end 131.064 70.0493) (width 0.25) (layer F.Cu) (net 3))
 (segment (start 140.358 50.601) (end 133.858 50.601) (width 0.25) (layer B.Cu) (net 3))
 (segment (start 132.668 58.928) (end 133.858 57.738) (width 0.25) (layer B.Cu) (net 3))
 (segment (start 133.858 57.738) (end 133.858 50.601) (width 0.25) (layer B.Cu) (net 3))
 (segment (start 131.064 69.4867) (end 131.3453 69.4867) (width 0.25) (layer F.Cu) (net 3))
 (segment (start 131.3453 69.4867) (end 132.668 68.164) (width 0.25) (layer F.Cu) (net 3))
 (segment (start 132.668 68.164) (end 132.668 58.928) (width 0.25) (layer F.Cu) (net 3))
 (segment (start 138.684 43.0853) (end 138.684 48.927) (width 0.25) (layer F.Cu) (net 3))
 (segment (start 138.684 48.927) (end 140.358 50.601) (width 0.25) (layer F.Cu) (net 3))
 (segment (start 128.778 45.72) (end 133.477 45.72) (width 0.25) (layer B.Cu) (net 4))
 (segment (start 133.477 45.72) (end 133.858 46.101) (width 0.25) (layer B.Cu) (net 4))
 (segment (start 140.358 46.101) (end 133.858 46.101) (width 0.25) (layer B.Cu) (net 4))
 (segment (start 128.524 41.91) (end 128.524 45.466) (width 0.25) (layer F.Cu) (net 4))
 (segment (start 128.524 45.466) (end 128.778 45.72) (width 0.25) (layer F.Cu) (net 4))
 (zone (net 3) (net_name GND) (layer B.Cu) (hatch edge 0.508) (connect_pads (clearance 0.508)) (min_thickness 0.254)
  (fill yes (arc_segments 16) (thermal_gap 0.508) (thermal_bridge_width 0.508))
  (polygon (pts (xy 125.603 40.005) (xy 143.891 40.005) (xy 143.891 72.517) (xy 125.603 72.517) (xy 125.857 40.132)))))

